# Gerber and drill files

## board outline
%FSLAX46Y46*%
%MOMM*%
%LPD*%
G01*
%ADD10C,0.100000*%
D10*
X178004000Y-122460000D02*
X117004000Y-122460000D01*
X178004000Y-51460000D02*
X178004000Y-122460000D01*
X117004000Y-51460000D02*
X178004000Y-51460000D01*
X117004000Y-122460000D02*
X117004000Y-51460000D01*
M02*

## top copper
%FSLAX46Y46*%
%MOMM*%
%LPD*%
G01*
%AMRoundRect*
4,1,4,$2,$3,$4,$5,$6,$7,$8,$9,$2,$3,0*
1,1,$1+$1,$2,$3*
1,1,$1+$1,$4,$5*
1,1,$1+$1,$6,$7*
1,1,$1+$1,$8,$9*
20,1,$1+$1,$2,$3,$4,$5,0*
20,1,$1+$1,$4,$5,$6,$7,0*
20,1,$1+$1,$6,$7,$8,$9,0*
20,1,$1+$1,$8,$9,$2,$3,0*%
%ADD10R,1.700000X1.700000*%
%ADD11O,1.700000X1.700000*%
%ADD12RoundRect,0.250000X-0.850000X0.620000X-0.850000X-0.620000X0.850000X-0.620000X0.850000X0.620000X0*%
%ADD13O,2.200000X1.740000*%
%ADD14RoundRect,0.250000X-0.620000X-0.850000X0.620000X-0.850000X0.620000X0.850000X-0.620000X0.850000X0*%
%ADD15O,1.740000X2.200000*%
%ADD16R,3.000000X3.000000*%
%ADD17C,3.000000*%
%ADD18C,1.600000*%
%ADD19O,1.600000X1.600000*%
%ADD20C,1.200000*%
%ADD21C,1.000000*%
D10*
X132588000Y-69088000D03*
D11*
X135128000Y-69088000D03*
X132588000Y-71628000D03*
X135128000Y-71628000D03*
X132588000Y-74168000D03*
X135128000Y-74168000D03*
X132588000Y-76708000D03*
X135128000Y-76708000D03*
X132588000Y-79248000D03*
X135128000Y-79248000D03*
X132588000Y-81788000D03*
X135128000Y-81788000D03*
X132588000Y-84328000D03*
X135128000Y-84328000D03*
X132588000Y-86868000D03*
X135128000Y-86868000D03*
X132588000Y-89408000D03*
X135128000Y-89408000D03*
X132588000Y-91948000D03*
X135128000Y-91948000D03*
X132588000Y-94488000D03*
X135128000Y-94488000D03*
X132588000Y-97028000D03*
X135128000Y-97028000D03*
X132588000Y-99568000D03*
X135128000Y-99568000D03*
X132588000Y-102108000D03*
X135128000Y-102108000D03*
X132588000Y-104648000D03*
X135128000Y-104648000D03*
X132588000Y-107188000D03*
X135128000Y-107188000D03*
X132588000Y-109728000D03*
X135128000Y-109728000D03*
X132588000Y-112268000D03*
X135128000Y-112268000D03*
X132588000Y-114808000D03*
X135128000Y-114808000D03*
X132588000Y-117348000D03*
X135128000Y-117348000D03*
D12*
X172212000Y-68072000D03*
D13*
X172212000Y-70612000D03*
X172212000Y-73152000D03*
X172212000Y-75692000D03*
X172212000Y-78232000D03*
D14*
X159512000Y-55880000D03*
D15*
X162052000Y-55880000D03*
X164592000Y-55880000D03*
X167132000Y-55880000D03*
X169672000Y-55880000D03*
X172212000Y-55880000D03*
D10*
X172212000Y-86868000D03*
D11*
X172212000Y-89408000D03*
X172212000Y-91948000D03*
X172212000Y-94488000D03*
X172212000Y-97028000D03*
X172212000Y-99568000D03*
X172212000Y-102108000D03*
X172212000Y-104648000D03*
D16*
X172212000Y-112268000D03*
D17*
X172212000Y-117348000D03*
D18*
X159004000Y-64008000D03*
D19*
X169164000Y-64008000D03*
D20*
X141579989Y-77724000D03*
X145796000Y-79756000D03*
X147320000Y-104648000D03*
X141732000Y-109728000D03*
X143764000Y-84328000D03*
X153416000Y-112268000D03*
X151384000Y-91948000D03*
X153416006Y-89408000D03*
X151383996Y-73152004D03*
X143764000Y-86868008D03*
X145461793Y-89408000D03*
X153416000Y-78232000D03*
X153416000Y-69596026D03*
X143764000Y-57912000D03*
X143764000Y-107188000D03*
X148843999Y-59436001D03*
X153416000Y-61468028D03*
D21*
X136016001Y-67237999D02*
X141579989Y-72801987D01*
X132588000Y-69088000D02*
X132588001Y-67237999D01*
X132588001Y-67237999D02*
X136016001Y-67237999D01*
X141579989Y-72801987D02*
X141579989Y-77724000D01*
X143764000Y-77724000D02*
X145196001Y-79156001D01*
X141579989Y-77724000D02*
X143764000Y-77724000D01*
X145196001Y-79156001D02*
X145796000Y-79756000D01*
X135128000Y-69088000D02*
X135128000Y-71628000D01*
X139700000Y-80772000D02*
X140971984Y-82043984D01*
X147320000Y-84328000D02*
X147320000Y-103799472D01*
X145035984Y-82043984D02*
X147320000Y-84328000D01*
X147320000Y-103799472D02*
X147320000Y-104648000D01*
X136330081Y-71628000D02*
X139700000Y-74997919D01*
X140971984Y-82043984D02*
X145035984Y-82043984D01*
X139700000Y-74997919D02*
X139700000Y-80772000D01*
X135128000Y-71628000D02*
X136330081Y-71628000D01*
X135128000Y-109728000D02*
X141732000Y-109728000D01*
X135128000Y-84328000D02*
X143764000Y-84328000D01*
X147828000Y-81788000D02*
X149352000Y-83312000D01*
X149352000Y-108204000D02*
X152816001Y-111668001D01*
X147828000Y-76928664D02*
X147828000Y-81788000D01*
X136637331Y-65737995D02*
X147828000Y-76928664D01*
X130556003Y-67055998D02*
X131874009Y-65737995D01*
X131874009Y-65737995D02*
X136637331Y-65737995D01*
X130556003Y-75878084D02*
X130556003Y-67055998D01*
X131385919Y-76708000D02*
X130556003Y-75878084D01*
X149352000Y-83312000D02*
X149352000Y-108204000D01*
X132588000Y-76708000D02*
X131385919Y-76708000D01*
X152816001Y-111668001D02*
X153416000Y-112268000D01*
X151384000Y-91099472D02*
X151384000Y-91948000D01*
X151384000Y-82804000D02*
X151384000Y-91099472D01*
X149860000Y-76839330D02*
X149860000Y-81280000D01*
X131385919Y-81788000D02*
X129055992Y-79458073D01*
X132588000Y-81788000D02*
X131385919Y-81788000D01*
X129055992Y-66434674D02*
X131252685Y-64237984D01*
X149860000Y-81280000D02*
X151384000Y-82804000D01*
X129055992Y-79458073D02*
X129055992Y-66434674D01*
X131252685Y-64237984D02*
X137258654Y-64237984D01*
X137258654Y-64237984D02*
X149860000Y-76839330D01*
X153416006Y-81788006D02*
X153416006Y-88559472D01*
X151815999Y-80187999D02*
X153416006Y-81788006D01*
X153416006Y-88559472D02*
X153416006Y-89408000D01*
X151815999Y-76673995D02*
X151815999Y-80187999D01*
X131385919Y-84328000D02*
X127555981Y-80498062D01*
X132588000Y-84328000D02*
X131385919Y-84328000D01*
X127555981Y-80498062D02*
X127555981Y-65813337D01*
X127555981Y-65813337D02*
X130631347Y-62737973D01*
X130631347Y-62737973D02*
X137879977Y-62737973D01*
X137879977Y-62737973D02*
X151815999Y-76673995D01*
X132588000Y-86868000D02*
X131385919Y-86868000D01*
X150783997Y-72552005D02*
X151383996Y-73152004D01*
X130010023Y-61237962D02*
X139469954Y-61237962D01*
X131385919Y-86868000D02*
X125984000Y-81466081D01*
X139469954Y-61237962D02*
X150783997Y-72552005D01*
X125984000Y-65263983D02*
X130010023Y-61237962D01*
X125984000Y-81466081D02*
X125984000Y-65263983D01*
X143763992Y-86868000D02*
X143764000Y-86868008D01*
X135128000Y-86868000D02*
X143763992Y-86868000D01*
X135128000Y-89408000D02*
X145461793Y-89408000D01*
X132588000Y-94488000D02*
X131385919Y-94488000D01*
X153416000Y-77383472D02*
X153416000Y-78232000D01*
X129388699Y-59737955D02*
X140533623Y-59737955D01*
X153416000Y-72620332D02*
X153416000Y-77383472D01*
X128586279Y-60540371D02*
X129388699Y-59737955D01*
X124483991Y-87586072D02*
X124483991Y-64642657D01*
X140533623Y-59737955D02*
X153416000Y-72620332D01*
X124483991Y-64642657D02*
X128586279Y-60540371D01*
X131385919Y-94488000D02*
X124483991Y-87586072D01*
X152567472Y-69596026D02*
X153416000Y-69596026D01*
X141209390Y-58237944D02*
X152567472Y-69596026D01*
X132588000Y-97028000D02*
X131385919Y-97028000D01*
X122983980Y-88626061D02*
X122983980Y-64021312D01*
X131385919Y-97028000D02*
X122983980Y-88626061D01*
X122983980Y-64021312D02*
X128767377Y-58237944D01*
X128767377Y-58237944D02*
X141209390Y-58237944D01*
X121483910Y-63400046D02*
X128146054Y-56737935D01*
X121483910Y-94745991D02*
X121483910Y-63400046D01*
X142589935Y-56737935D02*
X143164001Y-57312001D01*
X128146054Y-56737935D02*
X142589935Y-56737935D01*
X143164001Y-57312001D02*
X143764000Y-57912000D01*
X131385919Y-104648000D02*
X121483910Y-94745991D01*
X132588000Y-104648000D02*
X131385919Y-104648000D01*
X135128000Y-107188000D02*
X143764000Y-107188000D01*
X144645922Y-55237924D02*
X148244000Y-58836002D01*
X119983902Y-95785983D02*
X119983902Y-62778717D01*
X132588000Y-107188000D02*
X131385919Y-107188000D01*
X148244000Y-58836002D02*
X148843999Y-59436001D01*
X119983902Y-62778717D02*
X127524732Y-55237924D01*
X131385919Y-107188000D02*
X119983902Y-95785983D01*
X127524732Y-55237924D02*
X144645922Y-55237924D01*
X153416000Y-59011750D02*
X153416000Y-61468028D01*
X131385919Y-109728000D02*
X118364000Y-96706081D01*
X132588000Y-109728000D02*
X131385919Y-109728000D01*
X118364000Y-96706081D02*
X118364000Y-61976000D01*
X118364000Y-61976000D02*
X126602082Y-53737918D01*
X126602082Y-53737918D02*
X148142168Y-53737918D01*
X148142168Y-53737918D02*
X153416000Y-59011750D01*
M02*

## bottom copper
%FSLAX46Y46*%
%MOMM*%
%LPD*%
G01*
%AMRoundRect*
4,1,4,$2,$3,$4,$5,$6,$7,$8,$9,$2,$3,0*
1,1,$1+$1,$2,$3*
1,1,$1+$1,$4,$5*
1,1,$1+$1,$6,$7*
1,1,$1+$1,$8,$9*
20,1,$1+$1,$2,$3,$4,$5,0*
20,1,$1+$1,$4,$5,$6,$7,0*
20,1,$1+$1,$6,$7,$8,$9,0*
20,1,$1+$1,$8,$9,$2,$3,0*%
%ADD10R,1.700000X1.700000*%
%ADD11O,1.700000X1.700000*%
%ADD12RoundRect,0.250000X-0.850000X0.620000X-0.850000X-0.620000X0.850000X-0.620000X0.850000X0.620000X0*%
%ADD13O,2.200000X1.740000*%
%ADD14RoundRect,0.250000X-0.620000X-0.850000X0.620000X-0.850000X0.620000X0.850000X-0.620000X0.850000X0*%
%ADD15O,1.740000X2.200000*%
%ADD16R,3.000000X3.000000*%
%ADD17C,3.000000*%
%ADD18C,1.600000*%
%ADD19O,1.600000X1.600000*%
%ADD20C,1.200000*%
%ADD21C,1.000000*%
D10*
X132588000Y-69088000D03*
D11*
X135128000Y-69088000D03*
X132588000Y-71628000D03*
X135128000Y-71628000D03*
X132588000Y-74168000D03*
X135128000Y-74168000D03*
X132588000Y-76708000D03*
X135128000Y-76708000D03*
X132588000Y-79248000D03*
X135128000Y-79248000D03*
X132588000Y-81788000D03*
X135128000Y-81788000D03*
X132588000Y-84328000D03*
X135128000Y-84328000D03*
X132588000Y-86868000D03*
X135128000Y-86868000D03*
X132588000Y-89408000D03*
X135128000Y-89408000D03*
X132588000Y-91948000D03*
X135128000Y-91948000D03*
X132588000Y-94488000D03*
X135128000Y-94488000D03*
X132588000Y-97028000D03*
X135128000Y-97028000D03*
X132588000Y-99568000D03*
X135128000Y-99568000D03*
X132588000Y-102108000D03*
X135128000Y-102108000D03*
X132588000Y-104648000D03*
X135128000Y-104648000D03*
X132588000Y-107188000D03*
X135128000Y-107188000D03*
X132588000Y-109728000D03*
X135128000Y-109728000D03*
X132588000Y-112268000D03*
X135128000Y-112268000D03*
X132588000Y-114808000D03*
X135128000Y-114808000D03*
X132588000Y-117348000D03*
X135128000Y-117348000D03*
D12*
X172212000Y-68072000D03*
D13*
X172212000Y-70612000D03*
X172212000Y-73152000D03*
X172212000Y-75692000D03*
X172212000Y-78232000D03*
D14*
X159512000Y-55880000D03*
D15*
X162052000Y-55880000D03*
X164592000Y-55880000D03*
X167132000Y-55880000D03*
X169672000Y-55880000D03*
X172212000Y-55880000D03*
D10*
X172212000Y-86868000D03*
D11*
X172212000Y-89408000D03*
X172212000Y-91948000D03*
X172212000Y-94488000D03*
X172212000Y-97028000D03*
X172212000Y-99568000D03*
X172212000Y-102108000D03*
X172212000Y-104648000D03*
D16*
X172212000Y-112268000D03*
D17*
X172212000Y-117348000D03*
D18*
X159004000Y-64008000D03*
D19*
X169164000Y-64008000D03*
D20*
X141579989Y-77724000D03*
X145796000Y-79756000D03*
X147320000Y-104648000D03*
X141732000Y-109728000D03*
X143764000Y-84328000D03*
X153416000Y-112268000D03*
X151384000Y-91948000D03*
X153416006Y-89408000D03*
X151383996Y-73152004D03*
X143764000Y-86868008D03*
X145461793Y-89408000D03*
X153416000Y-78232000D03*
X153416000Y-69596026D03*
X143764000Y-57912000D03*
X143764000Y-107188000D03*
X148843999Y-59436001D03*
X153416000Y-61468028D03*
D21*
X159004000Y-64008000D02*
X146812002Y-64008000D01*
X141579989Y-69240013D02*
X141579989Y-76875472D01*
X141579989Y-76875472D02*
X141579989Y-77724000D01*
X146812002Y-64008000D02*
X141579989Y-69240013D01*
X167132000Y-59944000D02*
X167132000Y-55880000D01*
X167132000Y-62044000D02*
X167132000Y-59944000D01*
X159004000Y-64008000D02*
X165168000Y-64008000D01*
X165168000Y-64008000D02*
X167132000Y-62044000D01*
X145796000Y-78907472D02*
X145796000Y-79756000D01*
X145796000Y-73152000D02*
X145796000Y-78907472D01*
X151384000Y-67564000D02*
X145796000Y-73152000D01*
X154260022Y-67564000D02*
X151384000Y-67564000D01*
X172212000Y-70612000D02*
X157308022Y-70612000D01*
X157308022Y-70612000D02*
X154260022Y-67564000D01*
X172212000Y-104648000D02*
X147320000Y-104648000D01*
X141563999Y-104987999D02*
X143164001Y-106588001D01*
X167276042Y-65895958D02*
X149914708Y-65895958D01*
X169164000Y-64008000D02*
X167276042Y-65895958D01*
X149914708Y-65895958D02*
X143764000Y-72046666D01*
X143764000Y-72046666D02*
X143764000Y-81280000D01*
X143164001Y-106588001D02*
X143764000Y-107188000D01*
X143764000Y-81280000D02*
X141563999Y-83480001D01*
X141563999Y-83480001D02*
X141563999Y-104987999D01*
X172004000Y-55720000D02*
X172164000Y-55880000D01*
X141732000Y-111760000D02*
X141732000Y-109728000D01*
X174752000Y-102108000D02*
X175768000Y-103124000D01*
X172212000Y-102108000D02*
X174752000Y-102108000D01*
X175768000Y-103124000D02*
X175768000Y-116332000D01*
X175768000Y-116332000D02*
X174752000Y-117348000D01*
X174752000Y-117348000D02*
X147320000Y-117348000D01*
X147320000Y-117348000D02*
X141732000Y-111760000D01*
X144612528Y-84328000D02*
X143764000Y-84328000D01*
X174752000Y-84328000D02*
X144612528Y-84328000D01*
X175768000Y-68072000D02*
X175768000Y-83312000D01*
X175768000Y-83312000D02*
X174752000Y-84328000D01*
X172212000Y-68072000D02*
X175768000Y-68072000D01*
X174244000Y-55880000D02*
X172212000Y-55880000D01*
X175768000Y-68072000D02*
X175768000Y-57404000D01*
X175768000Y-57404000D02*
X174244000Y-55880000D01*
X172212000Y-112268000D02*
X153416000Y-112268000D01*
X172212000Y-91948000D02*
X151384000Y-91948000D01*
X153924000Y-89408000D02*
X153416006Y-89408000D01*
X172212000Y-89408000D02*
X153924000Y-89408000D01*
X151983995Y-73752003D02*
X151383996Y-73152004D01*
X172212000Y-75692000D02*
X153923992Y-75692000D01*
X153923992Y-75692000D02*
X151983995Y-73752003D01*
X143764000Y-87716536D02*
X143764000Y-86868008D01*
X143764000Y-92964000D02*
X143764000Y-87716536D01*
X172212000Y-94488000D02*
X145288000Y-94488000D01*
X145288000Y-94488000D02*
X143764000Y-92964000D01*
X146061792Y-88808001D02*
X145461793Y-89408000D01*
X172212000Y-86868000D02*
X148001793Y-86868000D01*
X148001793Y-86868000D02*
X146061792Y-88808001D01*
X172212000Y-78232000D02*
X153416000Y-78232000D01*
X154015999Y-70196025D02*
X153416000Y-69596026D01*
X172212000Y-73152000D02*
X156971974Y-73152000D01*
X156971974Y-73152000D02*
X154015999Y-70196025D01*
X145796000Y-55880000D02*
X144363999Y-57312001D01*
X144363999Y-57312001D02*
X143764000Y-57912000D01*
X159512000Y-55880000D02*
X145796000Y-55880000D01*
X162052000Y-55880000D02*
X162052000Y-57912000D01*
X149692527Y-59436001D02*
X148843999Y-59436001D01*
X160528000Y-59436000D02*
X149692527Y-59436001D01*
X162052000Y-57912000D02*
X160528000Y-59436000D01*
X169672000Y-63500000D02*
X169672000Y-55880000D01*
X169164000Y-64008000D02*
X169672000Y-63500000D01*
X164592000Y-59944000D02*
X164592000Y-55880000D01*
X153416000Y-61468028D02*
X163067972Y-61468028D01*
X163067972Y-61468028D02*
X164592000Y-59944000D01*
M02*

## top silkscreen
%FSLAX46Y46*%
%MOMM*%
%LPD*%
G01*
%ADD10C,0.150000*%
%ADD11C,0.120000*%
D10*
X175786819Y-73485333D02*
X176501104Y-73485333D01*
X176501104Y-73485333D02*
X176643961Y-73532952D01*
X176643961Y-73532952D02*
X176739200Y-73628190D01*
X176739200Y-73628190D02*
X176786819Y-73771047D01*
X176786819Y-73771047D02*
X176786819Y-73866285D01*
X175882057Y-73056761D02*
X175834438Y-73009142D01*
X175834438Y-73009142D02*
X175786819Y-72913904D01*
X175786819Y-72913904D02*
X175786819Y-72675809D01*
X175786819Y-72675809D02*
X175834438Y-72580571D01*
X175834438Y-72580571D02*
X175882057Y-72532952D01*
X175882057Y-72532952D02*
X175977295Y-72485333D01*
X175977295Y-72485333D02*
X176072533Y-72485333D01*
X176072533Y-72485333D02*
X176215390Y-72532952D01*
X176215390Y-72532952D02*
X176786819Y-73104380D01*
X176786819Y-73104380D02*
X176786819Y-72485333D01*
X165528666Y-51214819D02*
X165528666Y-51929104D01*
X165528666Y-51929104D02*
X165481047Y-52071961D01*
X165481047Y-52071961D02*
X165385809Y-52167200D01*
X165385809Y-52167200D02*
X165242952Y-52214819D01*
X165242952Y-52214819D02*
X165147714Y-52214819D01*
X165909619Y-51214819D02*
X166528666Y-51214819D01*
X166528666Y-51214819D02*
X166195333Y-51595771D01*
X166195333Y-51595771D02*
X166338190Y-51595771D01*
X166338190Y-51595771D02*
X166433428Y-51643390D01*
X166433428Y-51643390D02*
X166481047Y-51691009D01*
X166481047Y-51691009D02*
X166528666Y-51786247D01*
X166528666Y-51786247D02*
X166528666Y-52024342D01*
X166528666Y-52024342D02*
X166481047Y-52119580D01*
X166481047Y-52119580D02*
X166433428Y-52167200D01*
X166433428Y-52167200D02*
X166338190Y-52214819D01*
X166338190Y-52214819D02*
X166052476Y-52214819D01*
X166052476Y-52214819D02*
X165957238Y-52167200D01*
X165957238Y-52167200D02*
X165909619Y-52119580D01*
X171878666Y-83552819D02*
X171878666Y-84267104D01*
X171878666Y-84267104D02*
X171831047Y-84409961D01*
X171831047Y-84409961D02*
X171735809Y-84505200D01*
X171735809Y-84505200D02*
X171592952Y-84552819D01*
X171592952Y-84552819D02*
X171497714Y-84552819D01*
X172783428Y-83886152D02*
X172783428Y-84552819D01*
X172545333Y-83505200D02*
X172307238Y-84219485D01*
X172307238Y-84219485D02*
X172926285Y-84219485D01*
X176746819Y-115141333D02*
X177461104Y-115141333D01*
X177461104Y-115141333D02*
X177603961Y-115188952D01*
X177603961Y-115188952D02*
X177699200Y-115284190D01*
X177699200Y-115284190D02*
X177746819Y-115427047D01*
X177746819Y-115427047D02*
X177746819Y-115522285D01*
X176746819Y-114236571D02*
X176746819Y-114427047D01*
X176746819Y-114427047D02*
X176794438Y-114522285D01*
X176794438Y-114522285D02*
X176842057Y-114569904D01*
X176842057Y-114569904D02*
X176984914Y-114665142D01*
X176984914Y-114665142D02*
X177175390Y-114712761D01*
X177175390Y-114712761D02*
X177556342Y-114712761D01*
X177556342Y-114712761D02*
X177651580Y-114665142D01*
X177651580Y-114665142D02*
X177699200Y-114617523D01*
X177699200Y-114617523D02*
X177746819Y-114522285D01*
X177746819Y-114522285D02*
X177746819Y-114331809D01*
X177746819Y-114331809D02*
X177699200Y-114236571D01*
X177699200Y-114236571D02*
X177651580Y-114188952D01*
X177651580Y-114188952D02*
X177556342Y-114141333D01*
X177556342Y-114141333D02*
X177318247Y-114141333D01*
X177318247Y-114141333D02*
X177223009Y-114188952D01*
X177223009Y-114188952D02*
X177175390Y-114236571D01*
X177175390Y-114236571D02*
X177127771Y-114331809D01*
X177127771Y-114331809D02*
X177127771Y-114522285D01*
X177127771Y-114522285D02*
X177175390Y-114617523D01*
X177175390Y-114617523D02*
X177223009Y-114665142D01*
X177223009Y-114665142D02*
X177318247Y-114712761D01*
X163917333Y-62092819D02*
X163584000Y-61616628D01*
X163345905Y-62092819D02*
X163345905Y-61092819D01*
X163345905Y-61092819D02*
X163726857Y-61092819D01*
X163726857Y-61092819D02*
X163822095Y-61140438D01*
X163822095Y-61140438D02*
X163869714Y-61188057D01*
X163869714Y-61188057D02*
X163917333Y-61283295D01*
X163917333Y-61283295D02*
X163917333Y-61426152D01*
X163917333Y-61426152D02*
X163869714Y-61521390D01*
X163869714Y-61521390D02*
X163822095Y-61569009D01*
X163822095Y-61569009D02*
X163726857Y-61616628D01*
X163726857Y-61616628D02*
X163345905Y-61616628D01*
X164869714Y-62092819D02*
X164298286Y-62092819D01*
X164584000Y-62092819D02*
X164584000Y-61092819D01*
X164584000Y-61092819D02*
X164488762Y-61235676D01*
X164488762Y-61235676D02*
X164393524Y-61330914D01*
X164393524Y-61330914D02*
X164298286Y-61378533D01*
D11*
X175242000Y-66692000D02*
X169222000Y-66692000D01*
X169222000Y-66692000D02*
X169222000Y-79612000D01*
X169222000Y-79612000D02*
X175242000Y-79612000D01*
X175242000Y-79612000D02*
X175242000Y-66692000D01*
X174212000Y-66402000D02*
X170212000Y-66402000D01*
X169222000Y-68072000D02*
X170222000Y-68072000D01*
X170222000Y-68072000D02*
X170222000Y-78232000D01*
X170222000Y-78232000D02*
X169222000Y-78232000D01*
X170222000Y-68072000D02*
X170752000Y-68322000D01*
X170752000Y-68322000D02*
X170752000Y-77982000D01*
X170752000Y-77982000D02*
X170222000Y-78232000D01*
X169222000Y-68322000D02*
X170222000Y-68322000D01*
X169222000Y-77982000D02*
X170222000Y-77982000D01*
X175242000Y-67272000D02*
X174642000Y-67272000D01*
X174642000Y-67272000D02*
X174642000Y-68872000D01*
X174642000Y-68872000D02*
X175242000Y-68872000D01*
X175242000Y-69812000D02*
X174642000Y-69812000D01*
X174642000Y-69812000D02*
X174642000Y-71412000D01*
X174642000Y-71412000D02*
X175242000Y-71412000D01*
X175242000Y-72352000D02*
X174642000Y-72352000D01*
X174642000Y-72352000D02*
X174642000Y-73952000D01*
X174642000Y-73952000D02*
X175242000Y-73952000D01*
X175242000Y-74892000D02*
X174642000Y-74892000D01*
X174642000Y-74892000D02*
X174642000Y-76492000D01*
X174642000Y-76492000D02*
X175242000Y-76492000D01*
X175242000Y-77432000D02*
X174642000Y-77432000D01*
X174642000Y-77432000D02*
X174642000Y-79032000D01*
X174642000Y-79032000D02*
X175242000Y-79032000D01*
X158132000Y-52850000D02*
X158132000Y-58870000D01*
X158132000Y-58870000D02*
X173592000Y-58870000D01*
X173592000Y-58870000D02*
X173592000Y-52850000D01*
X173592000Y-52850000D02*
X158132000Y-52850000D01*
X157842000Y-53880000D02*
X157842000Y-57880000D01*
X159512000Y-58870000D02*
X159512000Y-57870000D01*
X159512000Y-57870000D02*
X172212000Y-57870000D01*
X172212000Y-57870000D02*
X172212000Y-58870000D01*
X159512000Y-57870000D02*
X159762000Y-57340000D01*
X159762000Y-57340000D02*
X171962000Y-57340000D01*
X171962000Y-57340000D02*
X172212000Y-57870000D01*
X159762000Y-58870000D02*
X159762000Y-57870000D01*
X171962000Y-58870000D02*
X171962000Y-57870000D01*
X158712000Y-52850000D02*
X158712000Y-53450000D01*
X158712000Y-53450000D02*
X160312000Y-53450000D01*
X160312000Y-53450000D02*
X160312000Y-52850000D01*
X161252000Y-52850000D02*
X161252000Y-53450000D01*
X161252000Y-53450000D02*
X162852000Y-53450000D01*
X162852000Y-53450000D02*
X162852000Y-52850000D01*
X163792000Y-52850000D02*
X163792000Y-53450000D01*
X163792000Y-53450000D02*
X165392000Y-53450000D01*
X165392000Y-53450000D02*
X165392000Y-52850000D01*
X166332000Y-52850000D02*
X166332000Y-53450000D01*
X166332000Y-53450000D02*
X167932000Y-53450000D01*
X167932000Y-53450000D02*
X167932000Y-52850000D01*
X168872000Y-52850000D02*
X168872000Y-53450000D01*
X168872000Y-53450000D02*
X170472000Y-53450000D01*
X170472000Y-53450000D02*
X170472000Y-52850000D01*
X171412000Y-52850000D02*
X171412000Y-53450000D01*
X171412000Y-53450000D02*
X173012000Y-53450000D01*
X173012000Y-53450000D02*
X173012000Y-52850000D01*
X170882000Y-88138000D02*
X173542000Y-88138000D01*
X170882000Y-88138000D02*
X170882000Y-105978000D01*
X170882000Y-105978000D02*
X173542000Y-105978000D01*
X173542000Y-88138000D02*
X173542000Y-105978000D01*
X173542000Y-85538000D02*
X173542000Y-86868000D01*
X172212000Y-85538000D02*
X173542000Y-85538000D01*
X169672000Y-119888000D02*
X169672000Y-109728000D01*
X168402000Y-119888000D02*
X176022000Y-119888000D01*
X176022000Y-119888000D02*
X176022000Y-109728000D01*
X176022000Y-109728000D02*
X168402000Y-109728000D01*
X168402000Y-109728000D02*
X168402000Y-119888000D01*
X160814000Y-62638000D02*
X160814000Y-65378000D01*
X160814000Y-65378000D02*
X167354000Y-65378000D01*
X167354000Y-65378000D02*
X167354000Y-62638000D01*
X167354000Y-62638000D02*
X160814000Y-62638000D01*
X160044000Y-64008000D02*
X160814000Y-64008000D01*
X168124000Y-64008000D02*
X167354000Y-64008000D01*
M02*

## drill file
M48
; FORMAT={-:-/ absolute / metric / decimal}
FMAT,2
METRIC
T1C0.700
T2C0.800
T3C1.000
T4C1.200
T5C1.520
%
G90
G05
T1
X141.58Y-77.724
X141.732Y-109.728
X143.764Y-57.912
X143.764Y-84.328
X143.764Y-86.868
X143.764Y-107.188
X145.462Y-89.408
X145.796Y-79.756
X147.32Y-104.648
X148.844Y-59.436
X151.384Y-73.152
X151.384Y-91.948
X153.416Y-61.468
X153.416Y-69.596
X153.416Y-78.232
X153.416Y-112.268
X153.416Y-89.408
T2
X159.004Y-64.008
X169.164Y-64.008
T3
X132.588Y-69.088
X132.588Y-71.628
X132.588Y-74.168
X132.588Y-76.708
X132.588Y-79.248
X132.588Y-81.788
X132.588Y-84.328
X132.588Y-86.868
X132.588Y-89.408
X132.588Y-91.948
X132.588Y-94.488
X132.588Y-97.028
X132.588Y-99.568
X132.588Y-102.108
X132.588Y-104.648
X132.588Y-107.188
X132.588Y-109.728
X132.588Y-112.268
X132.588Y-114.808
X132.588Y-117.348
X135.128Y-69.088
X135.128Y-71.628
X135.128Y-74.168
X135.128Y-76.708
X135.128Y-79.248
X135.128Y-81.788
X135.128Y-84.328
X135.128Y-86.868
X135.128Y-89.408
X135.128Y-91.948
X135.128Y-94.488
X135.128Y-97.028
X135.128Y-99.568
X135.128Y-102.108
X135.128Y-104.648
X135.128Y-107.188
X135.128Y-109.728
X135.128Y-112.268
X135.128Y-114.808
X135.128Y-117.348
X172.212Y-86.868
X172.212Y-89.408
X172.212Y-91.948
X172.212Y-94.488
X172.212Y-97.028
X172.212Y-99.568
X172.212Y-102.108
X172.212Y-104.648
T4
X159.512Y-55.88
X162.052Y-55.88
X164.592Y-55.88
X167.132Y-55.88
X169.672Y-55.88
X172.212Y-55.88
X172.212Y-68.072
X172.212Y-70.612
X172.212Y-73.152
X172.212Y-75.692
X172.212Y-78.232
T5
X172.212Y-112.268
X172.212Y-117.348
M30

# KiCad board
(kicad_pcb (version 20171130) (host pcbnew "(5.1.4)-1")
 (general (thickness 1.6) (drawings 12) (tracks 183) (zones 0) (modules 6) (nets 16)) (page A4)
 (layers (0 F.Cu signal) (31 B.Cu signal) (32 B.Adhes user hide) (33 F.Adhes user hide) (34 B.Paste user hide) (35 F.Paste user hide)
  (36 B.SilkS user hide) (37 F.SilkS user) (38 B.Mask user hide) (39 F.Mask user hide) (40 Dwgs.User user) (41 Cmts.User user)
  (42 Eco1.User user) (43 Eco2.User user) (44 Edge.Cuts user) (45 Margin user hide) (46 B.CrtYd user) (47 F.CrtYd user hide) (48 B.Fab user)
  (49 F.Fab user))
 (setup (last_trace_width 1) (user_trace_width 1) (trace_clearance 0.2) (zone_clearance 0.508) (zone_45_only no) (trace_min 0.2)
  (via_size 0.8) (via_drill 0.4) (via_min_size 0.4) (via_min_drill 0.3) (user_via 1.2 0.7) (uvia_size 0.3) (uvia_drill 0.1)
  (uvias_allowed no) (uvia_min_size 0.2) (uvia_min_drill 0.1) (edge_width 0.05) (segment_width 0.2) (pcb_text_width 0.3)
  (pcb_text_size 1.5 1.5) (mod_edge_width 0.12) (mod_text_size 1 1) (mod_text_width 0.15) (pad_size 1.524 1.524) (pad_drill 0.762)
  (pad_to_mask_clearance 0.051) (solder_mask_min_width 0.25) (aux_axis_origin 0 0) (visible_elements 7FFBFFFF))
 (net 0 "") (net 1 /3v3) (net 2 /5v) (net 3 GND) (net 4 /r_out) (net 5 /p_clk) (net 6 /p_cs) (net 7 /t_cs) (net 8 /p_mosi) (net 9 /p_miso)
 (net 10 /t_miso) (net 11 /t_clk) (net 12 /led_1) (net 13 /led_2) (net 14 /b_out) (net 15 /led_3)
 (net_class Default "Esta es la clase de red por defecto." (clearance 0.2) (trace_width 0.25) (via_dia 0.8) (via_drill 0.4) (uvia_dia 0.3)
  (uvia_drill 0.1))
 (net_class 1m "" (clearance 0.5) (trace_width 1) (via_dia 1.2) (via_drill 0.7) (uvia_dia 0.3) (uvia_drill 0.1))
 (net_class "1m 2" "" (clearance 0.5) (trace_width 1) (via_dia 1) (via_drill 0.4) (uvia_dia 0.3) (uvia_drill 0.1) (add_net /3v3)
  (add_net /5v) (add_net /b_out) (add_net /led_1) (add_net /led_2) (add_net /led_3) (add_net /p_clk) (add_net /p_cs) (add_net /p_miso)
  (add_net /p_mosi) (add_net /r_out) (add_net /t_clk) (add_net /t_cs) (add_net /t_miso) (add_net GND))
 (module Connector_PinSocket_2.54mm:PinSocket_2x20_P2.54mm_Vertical (layer B.Cu) (at 132.588 69.088 180)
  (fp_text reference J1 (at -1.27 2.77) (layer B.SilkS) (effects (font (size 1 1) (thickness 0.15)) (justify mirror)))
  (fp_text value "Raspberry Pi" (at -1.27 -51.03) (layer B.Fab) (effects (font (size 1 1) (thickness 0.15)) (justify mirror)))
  (pad 1 thru_hole rect (at 0 0 180) (size 1.7 1.7) (drill 1) (layers *.Cu *.Mask) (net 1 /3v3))
  (pad 2 thru_hole oval (at -2.54 0 180) (size 1.7 1.7) (drill 1) (layers *.Cu *.Mask) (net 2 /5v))
  (pad 3 thru_hole oval (at 0 -2.54 180) (size 1.7 1.7) (drill 1) (layers *.Cu *.Mask))
  (pad 4 thru_hole oval (at -2.54 -2.54 180) (size 1.7 1.7) (drill 1) (layers *.Cu *.Mask) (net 2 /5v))
  (pad 5 thru_hole oval (at 0 -5.08 180) (size 1.7 1.7) (drill 1) (layers *.Cu *.Mask))
  (pad 6 thru_hole oval (at -2.54 -5.08 180) (size 1.7 1.7) (drill 1) (layers *.Cu *.Mask) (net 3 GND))
  (pad 7 thru_hole oval (at 0 -7.62 180) (size 1.7 1.7) (drill 1) (layers *.Cu *.Mask) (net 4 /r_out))
  (pad 8 thru_hole oval (at -2.54 -7.62 180) (size 1.7 1.7) (drill 1) (layers *.Cu *.Mask))
  (pad 9 thru_hole oval (at 0 -10.16 180) (size 1.7 1.7) (drill 1) (layers *.Cu *.Mask))
  (pad 10 thru_hole oval (at -2.54 -10.16 180) (size 1.7 1.7) (drill 1) (layers *.Cu *.Mask))
  (pad 11 thru_hole oval (at 0 -12.7 180) (size 1.7 1.7) (drill 1) (layers *.Cu *.Mask) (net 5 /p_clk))
  (pad 12 thru_hole oval (at -2.54 -12.7 180) (size 1.7 1.7) (drill 1) (layers *.Cu *.Mask))
  (pad 13 thru_hole oval (at 0 -15.24 180) (size 1.7 1.7) (drill 1) (layers *.Cu *.Mask) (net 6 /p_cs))
  (pad 14 thru_hole oval (at -2.54 -15.24 180) (size 1.7 1.7) (drill 1) (layers *.Cu *.Mask) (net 3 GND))
  (pad 15 thru_hole oval (at 0 -17.78 180) (size 1.7 1.7) (drill 1) (layers *.Cu *.Mask) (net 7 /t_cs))
  (pad 16 thru_hole oval (at -2.54 -17.78 180) (size 1.7 1.7) (drill 1) (layers *.Cu *.Mask) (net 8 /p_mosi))
  (pad 17 thru_hole oval (at 0 -20.32 180) (size 1.7 1.7) (drill 1) (layers *.Cu *.Mask))
  (pad 18 thru_hole oval (at -2.54 -20.32 180) (size 1.7 1.7) (drill 1) (layers *.Cu *.Mask) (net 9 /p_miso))
  (pad 19 thru_hole oval (at 0 -22.86 180) (size 1.7 1.7) (drill 1) (layers *.Cu *.Mask))
  (pad 20 thru_hole oval (at -2.54 -22.86 180) (size 1.7 1.7) (drill 1) (layers *.Cu *.Mask) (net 3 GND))
  (pad 21 thru_hole oval (at 0 -25.4 180) (size 1.7 1.7) (drill 1) (layers *.Cu *.Mask) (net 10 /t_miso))
  (pad 22 thru_hole oval (at -2.54 -25.4 180) (size 1.7 1.7) (drill 1) (layers *.Cu *.Mask))
  (pad 23 thru_hole oval (at 0 -27.94 180) (size 1.7 1.7) (drill 1) (layers *.Cu *.Mask) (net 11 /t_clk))
  (pad 24 thru_hole oval (at -2.54 -27.94 180) (size 1.7 1.7) (drill 1) (layers *.Cu *.Mask))
  (pad 25 thru_hole oval (at 0 -30.48 180) (size 1.7 1.7) (drill 1) (layers *.Cu *.Mask))
  (pad 26 thru_hole oval (at -2.54 -30.48 180) (size 1.7 1.7) (drill 1) (layers *.Cu *.Mask))
  (pad 27 thru_hole oval (at 0 -33.02 180) (size 1.7 1.7) (drill 1) (layers *.Cu *.Mask))
  (pad 28 thru_hole oval (at -2.54 -33.02 180) (size 1.7 1.7) (drill 1) (layers *.Cu *.Mask))
  (pad 29 thru_hole oval (at 0 -35.56 180) (size 1.7 1.7) (drill 1) (layers *.Cu *.Mask) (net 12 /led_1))
  (pad 30 thru_hole oval (at -2.54 -35.56 180) (size 1.7 1.7) (drill 1) (layers *.Cu *.Mask) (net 3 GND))
  (pad 31 thru_hole oval (at 0 -38.1 180) (size 1.7 1.7) (drill 1) (layers *.Cu *.Mask) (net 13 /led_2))
  (pad 32 thru_hole oval (at -2.54 -38.1 180) (size 1.7 1.7) (drill 1) (layers *.Cu *.Mask) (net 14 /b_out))
  (pad 33 thru_hole oval (at 0 -40.64 180) (size 1.7 1.7) (drill 1) (layers *.Cu *.Mask) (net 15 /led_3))
  (pad 34 thru_hole oval (at -2.54 -40.64 180) (size 1.7 1.7) (drill 1) (layers *.Cu *.Mask) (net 3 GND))
  (pad 35 thru_hole oval (at 0 -43.18 180) (size 1.7 1.7) (drill 1) (layers *.Cu *.Mask))
  (pad 36 thru_hole oval (at -2.54 -43.18 180) (size 1.7 1.7) (drill 1) (layers *.Cu *.Mask))
  (pad 37 thru_hole oval (at 0 -45.72 180) (size 1.7 1.7) (drill 1) (layers *.Cu *.Mask))
  (pad 38 thru_hole oval (at -2.54 -45.72 180) (size 1.7 1.7) (drill 1) (layers *.Cu *.Mask))
  (pad 39 thru_hole oval (at 0 -48.26 180) (size 1.7 1.7) (drill 1) (layers *.Cu *.Mask))
  (pad 40 thru_hole oval (at -2.54 -48.26 180) (size 1.7 1.7) (drill 1) (layers *.Cu *.Mask)))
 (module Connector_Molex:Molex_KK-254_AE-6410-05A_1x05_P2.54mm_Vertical (layer F.Cu) (at 172.212 68.072 270)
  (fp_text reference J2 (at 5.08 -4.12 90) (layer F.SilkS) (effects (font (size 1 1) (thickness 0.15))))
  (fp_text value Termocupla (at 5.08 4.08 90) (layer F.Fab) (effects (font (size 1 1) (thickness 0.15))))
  (fp_line (start -1.38 -3.03) (end -1.38 2.99) (layer F.SilkS) (width 0.12))
  (fp_line (start -1.38 2.99) (end 11.54 2.99) (layer F.SilkS) (width 0.12))
  (fp_line (start 11.54 2.99) (end 11.54 -3.03) (layer F.SilkS) (width 0.12))
  (fp_line (start 11.54 -3.03) (end -1.38 -3.03) (layer F.SilkS) (width 0.12))
  (fp_line (start -1.67 -2) (end -1.67 2) (layer F.SilkS) (width 0.12))
  (fp_line (start 0 2.99) (end 0 1.99) (layer F.SilkS) (width 0.12))
  (fp_line (start 0 1.99) (end 10.16 1.99) (layer F.SilkS) (width 0.12))
  (fp_line (start 10.16 1.99) (end 10.16 2.99) (layer F.SilkS) (width 0.12))
  (fp_line (start 0 1.99) (end 0.25 1.46) (layer F.SilkS) (width 0.12))
  (fp_line (start 0.25 1.46) (end 9.91 1.46) (layer F.SilkS) (width 0.12))
  (fp_line (start 9.91 1.46) (end 10.16 1.99) (layer F.SilkS) (width 0.12))
  (fp_line (start 0.25 2.99) (end 0.25 1.99) (layer F.SilkS) (width 0.12))
  (fp_line (start 9.91 2.99) (end 9.91 1.99) (layer F.SilkS) (width 0.12))
  (fp_line (start -0.8 -3.03) (end -0.8 -2.43) (layer F.SilkS) (width 0.12))
  (fp_line (start -0.8 -2.43) (end 0.8 -2.43) (layer F.SilkS) (width 0.12))
  (fp_line (start 0.8 -2.43) (end 0.8 -3.03) (layer F.SilkS) (width 0.12))
  (fp_line (start 1.74 -3.03) (end 1.74 -2.43) (layer F.SilkS) (width 0.12))
  (fp_line (start 1.74 -2.43) (end 3.34 -2.43) (layer F.SilkS) (width 0.12))
  (fp_line (start 3.34 -2.43) (end 3.34 -3.03) (layer F.SilkS) (width 0.12))
  (fp_line (start 4.28 -3.03) (end 4.28 -2.43) (layer F.SilkS) (width 0.12))
  (fp_line (start 4.28 -2.43) (end 5.88 -2.43) (layer F.SilkS) (width 0.12))
  (fp_line (start 5.88 -2.43) (end 5.88 -3.03) (layer F.SilkS) (width 0.12))
  (fp_line (start 6.82 -3.03) (end 6.82 -2.43) (layer F.SilkS) (width 0.12))
  (fp_line (start 6.82 -2.43) (end 8.42 -2.43) (layer F.SilkS) (width 0.12))
  (fp_line (start 8.42 -2.43) (end 8.42 -3.03) (layer F.SilkS) (width 0.12))
  (fp_line (start 9.36 -3.03) (end 9.36 -2.43) (layer F.SilkS) (width 0.12))
  (fp_line (start 9.36 -2.43) (end 10.96 -2.43) (layer F.SilkS) (width 0.12))
  (fp_line (start 10.96 -2.43) (end 10.96 -3.03) (layer F.SilkS) (width 0.12))
  (pad 1 thru_hole roundrect (at 0 0 270) (size 1.74 2.2) (drill 1.2) (layers *.Cu *.Mask) (roundrect_rratio 0.143678) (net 3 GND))
  (pad 2 thru_hole oval (at 2.54 0 270) (size 1.74 2.2) (drill 1.2) (layers *.Cu *.Mask) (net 1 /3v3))
  (pad 3 thru_hole oval (at 5.08 0 270) (size 1.74 2.2) (drill 1.2) (layers *.Cu *.Mask) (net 11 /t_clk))
  (pad 4 thru_hole oval (at 7.62 0 270) (size 1.74 2.2) (drill 1.2) (layers *.Cu *.Mask) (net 7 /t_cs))
  (pad 5 thru_hole oval (at 10.16 0 270) (size 1.74 2.2) (drill 1.2) (layers *.Cu *.Mask) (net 10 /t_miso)))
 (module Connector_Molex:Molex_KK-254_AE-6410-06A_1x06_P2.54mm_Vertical (layer F.Cu) (at 159.512 55.88)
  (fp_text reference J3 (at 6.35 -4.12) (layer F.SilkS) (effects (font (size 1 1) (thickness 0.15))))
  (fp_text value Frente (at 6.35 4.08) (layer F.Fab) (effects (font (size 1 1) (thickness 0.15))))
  (fp_line (start -1.38 -3.03) (end -1.38 2.99) (layer F.SilkS) (width 0.12))
  (fp_line (start -1.38 2.99) (end 14.08 2.99) (layer F.SilkS) (width 0.12))
  (fp_line (start 14.08 2.99) (end 14.08 -3.03) (layer F.SilkS) (width 0.12))
  (fp_line (start 14.08 -3.03) (end -1.38 -3.03) (layer F.SilkS) (width 0.12))
  (fp_line (start -1.67 -2) (end -1.67 2) (layer F.SilkS) (width 0.12))
  (fp_line (start 0 2.99) (end 0 1.99) (layer F.SilkS) (width 0.12))
  (fp_line (start 0 1.99) (end 12.7 1.99) (layer F.SilkS) (width 0.12))
  (fp_line (start 12.7 1.99) (end 12.7 2.99) (layer F.SilkS) (width 0.12))
  (fp_line (start 0 1.99) (end 0.25 1.46) (layer F.SilkS) (width 0.12))
  (fp_line (start 0.25 1.46) (end 12.45 1.46) (layer F.SilkS) (width 0.12))
  (fp_line (start 12.45 1.46) (end 12.7 1.99) (layer F.SilkS) (width 0.12))
  (fp_line (start 0.25 2.99) (end 0.25 1.99) (layer F.SilkS) (width 0.12))
  (fp_line (start 12.45 2.99) (end 12.45 1.99) (layer F.SilkS) (width 0.12))
  (fp_line (start -0.8 -3.03) (end -0.8 -2.43) (layer F.SilkS) (width 0.12))
  (fp_line (start -0.8 -2.43) (end 0.8 -2.43) (layer F.SilkS) (width 0.12))
  (fp_line (start 0.8 -2.43) (end 0.8 -3.03) (layer F.SilkS) (width 0.12))
  (fp_line (start 1.74 -3.03) (end 1.74 -2.43) (layer F.SilkS) (width 0.12))
  (fp_line (start 1.74 -2.43) (end 3.34 -2.43) (layer F.SilkS) (width 0.12))
  (fp_line (start 3.34 -2.43) (end 3.34 -3.03) (layer F.SilkS) (width 0.12))
  (fp_line (start 4.28 -3.03) (end 4.28 -2.43) (layer F.SilkS) (width 0.12))
  (fp_line (start 4.28 -2.43) (end 5.88 -2.43) (layer F.SilkS) (width 0.12))
  (fp_line (start 5.88 -2.43) (end 5.88 -3.03) (layer F.SilkS) (width 0.12))
  (fp_line (start 6.82 -3.03) (end 6.82 -2.43) (layer F.SilkS) (width 0.12))
  (fp_line (start 6.82 -2.43) (end 8.42 -2.43) (layer F.SilkS) (width 0.12))
  (fp_line (start 8.42 -2.43) (end 8.42 -3.03) (layer F.SilkS) (width 0.12))
  (fp_line (start 9.36 -3.03) (end 9.36 -2.43) (layer F.SilkS) (width 0.12))
  (fp_line (start 9.36 -2.43) (end 10.96 -2.43) (layer F.SilkS) (width 0.12))
  (fp_line (start 10.96 -2.43) (end 10.96 -3.03) (layer F.SilkS) (width 0.12))
  (fp_line (start 11.9 -3.03) (end 11.9 -2.43) (layer F.SilkS) (width 0.12))
  (fp_line (start 11.9 -2.43) (end 13.5 -2.43) (layer F.SilkS) (width 0.12))
  (fp_line (start 13.5 -2.43) (end 13.5 -3.03) (layer F.SilkS) (width 0.12))
  (pad 1 thru_hole roundrect (at 0 0) (size 1.74 2.2) (drill 1.2) (layers *.Cu *.Mask) (roundrect_rratio 0.143678) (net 12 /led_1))
  (pad 2 thru_hole oval (at 2.54 0) (size 1.74 2.2) (drill 1.2) (layers *.Cu *.Mask) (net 13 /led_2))
  (pad 3 thru_hole oval (at 5.08 0) (size 1.74 2.2) (drill 1.2) (layers *.Cu *.Mask) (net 15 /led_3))
  (pad 4 thru_hole oval (at 7.62 0) (size 1.74 2.2) (drill 1.2) (layers *.Cu *.Mask) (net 1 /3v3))
  (pad 5 thru_hole oval (at 10.16 0) (size 1.74 2.2) (drill 1.2) (layers *.Cu *.Mask) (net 14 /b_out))
  (pad 6 thru_hole oval (at 12.7 0) (size 1.74 2.2) (drill 1.2) (layers *.Cu *.Mask) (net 3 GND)))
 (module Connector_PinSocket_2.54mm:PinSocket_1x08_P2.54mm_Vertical (layer F.Cu) (at 172.212 86.868)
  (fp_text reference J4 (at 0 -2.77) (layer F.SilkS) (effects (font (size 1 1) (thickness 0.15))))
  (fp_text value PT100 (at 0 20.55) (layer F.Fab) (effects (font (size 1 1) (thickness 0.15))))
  (fp_line (start -1.33 1.27) (end 1.33 1.27) (layer F.SilkS) (width 0.12))
  (fp_line (start -1.33 1.27) (end -1.33 19.11) (layer F.SilkS) (width 0.12))
  (fp_line (start -1.33 19.11) (end 1.33 19.11) (layer F.SilkS) (width 0.12))
  (fp_line (start 1.33 1.27) (end 1.33 19.11) (layer F.SilkS) (width 0.12))
  (fp_line (start 1.33 -1.33) (end 1.33 0) (layer F.SilkS) (width 0.12))
  (fp_line (start 0 -1.33) (end 1.33 -1.33) (layer F.SilkS) (width 0.12))
  (pad 1 thru_hole rect (at 0 0) (size 1.7 1.7) (drill 1) (layers *.Cu *.Mask) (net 9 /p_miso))
  (pad 2 thru_hole oval (at 0 2.54) (size 1.7 1.7) (drill 1) (layers *.Cu *.Mask) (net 6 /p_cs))
  (pad 3 thru_hole oval (at 0 5.08) (size 1.7 1.7) (drill 1) (layers *.Cu *.Mask) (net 5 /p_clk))
  (pad 4 thru_hole oval (at 0 7.62) (size 1.7 1.7) (drill 1) (layers *.Cu *.Mask) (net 8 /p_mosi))
  (pad 5 thru_hole oval (at 0 10.16) (size 1.7 1.7) (drill 1) (layers *.Cu *.Mask))
  (pad 6 thru_hole oval (at 0 12.7) (size 1.7 1.7) (drill 1) (layers *.Cu *.Mask))
  (pad 7 thru_hole oval (at 0 15.24) (size 1.7 1.7) (drill 1) (layers *.Cu *.Mask) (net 3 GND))
  (pad 8 thru_hole oval (at 0 17.78) (size 1.7 1.7) (drill 1) (layers *.Cu *.Mask) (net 2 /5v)))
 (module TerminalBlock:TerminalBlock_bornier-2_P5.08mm (layer F.Cu) (at 172.212 112.268 270)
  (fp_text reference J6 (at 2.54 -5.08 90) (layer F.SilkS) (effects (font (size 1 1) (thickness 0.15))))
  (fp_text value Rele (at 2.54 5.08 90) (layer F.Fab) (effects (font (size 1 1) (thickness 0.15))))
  (fp_line (start 7.62 2.54) (end -2.54 2.54) (layer F.SilkS) (width 0.12))
  (fp_line (start 7.62 3.81) (end 7.62 -3.81) (layer F.SilkS) (width 0.12))
  (fp_line (start 7.62 -3.81) (end -2.54 -3.81) (layer F.SilkS) (width 0.12))
  (fp_line (start -2.54 -3.81) (end -2.54 3.81) (layer F.SilkS) (width 0.12))
  (fp_line (start -2.54 3.81) (end 7.62 3.81) (layer F.SilkS) (width 0.12))
  (pad 1 thru_hole rect (at 0 0 270) (size 3 3) (drill 1.52) (layers *.Cu *.Mask) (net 4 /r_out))
  (pad 2 thru_hole circle (at 5.08 0 270) (size 3 3) (drill 1.52) (layers *.Cu *.Mask) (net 3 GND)))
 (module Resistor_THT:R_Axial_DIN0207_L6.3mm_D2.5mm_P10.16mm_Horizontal (layer F.Cu) (at 159.004 64.008)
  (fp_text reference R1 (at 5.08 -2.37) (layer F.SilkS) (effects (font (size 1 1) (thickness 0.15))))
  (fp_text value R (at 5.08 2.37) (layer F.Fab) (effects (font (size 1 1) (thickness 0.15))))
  (fp_line (start 1.81 -1.37) (end 1.81 1.37) (layer F.SilkS) (width 0.12))
  (fp_line (start 1.81 1.37) (end 8.35 1.37) (layer F.SilkS) (width 0.12))
  (fp_line (start 8.35 1.37) (end 8.35 -1.37) (layer F.SilkS) (width 0.12))
  (fp_line (start 8.35 -1.37) (end 1.81 -1.37) (layer F.SilkS) (width 0.12))
  (fp_line (start 1.04 0) (end 1.81 0) (layer F.SilkS) (width 0.12))
  (fp_line (start 9.12 0) (end 8.35 0) (layer F.SilkS) (width 0.12))
  (pad 1 thru_hole circle (at 0 0) (size 1.6 1.6) (drill 0.8) (layers *.Cu *.Mask) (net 1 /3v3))
  (pad 2 thru_hole oval (at 10.16 0) (size 1.6 1.6) (drill 0.8) (layers *.Cu *.Mask) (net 14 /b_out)))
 (gr_line (start 178.004 122.46) (end 117.004 122.46) (layer Edge.Cuts) (width 0.1))
 (gr_line (start 178.004 51.46) (end 178.004 122.46) (layer Edge.Cuts) (width 0.1))
 (gr_line (start 117.004 51.46) (end 178.004 51.46) (layer Edge.Cuts) (width 0.1))
 (gr_line (start 117.004 122.46) (end 117.004 51.46) (layer Edge.Cuts) (width 0.1))
 (segment (start 136.016001 67.237999) (end 141.579989 72.801987) (width 1) (layer F.Cu) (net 1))
 (segment (start 159.004 64.008) (end 146.812002 64.008) (width 1) (layer B.Cu) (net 1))
 (segment (start 141.579989 69.240013) (end 141.579989 76.875472) (width 1) (layer B.Cu) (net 1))
 (segment (start 141.579989 76.875472) (end 141.579989 77.724) (width 1) (layer B.Cu) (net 1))
 (segment (start 132.588 69.088) (end 132.588001 67.237999) (width 1) (layer F.Cu) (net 1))
 (segment (start 132.588001 67.237999) (end 136.016001 67.237999) (width 1) (layer F.Cu) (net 1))
 (segment (start 141.579989 72.801987) (end 141.579989 77.724) (width 1) (layer F.Cu) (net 1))
 (segment (start 146.812002 64.008) (end 141.579989 69.240013) (width 1) (layer B.Cu) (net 1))
 (via (at 141.579989 77.724) (size 1.2) (drill 0.7) (layers F.Cu B.Cu) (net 1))
 (via (at 145.796 79.756) (size 1.2) (drill 0.7) (layers F.Cu B.Cu) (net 1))
 (segment (start 143.764 77.724) (end 145.196001 79.156001) (width 1) (layer F.Cu) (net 1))
 (segment (start 141.579989 77.724) (end 143.764 77.724) (width 1) (layer F.Cu) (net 1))
 (segment (start 145.196001 79.156001) (end 145.796 79.756) (width 1) (layer F.Cu) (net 1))
 (segment (start 167.132 59.944) (end 167.132 55.88) (width 1) (layer B.Cu) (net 1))
 (segment (start 167.132 62.044) (end 167.132 59.944) (width 1) (layer B.Cu) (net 1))
 (segment (start 159.004 64.008) (end 165.168 64.008) (width 1) (layer B.Cu) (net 1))
 (segment (start 165.168 64.008) (end 167.132 62.044) (width 1) (layer B.Cu) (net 1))
 (segment (start 145.796 78.907472) (end 145.796 79.756) (width 1) (layer B.Cu) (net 1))
 (segment (start 145.796 73.152) (end 145.796 78.907472) (width 1) (layer B.Cu) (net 1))
 (segment (start 151.384 67.564) (end 145.796 73.152) (width 1) (layer B.Cu) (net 1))
 (segment (start 154.260022 67.564) (end 151.384 67.564) (width 1) (layer B.Cu) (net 1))
 (segment (start 172.212 70.612) (end 157.308022 70.612) (width 1) (layer B.Cu) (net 1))
 (segment (start 157.308022 70.612) (end 154.260022 67.564) (width 1) (layer B.Cu) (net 1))
 (segment (start 135.128 69.088) (end 135.128 71.628) (width 1) (layer F.Cu) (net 2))
 (via (at 147.32 104.648) (size 1.2) (drill 0.7) (layers F.Cu B.Cu) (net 2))
 (segment (start 139.7 80.772) (end 140.971984 82.043984) (width 1) (layer F.Cu) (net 2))
 (segment (start 147.32 84.328) (end 147.32 103.799472) (width 1) (layer F.Cu) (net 2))
 (segment (start 172.212 104.648) (end 147.32 104.648) (width 1) (layer B.Cu) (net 2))
 (segment (start 145.035984 82.043984) (end 147.32 84.328) (width 1) (layer F.Cu) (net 2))
 (segment (start 147.32 103.799472) (end 147.32 104.648) (width 1) (layer F.Cu) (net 2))
 (segment (start 136.330081 71.628) (end 139.7 74.997919) (width 1) (layer F.Cu) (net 2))
 (segment (start 140.971984 82.043984) (end 145.035984 82.043984) (width 1) (layer F.Cu) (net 2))
 (segment (start 139.7 74.997919) (end 139.7 80.772) (width 1) (layer F.Cu) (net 2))
 (segment (start 135.128 71.628) (end 136.330081 71.628) (width 1) (layer F.Cu) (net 2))
 (via (at 141.732 109.728) (size 1.2) (drill 0.7) (layers F.Cu B.Cu) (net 3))
 (segment (start 135.128 109.728) (end 141.732 109.728) (width 1) (layer F.Cu) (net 3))
 (via (at 143.764 84.328) (size 1.2) (drill 0.7) (layers F.Cu B.Cu) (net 3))
 (segment (start 135.128 84.328) (end 143.764 84.328) (width 1) (layer F.Cu) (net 3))
 (segment (start 147.828 81.788) (end 149.352 83.312) (width 1) (layer F.Cu) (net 4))
 (segment (start 149.352 108.204) (end 152.816001 111.668001) (width 1) (layer F.Cu) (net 4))
 (segment (start 147.828 76.928664) (end 147.828 81.788) (width 1) (layer F.Cu) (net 4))
 (segment (start 136.637331 65.737995) (end 147.828 76.928664) (width 1) (layer F.Cu) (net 4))
 (segment (start 130.556003 67.055998) (end 131.874009 65.737995) (width 1) (layer F.Cu) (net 4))
 (segment (start 131.874009 65.737995) (end 136.637331 65.737995) (width 1) (layer F.Cu) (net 4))
 (segment (start 130.556003 75.878084) (end 130.556003 67.055998) (width 1) (layer F.Cu) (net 4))
 (segment (start 131.385919 76.708) (end 130.556003 75.878084) (width 1) (layer F.Cu) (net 4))
 (segment (start 149.352 83.312) (end 149.352 108.204) (width 1) (layer F.Cu) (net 4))
 (segment (start 132.588 76.708) (end 131.385919 76.708) (width 1) (layer F.Cu) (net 4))
 (via (at 153.416 112.268) (size 1.2) (drill 0.7) (layers F.Cu B.Cu) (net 4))
 (segment (start 152.816001 111.668001) (end 153.416 112.268) (width 1) (layer F.Cu) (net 4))
 (via (at 151.384 91.948) (size 1.2) (drill 0.7) (layers F.Cu B.Cu) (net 5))
 (segment (start 151.384 91.099472) (end 151.384 91.948) (width 1) (layer F.Cu) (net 5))
 (segment (start 151.384 82.804) (end 151.384 91.099472) (width 1) (layer F.Cu) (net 5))
 (segment (start 149.86 76.83933) (end 149.86 81.28) (width 1) (layer F.Cu) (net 5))
 (segment (start 131.385919 81.788) (end 129.055992 79.458073) (width 1) (layer F.Cu) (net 5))
 (segment (start 132.588 81.788) (end 131.385919 81.788) (width 1) (layer F.Cu) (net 5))
 (segment (start 129.055992 66.434674) (end 131.252685 64.237984) (width 1) (layer F.Cu) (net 5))
 (segment (start 149.86 81.28) (end 151.384 82.804) (width 1) (layer F.Cu) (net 5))
 (segment (start 129.055992 79.458073) (end 129.055992 66.434674) (width 1) (layer F.Cu) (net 5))
 (segment (start 131.252685 64.237984) (end 137.258654 64.237984) (width 1) (layer F.Cu) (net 5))
 (segment (start 137.258654 64.237984) (end 149.86 76.83933) (width 1) (layer F.Cu) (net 5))
 (via (at 153.416006 89.408) (size 1.2) (drill 0.7) (layers F.Cu B.Cu) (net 6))
 (segment (start 153.416006 81.788006) (end 153.416006 88.559472) (width 1) (layer F.Cu) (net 6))
 (segment (start 151.815999 80.187999) (end 153.416006 81.788006) (width 1) (layer F.Cu) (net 6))
 (segment (start 153.416006 88.559472) (end 153.416006 89.408) (width 1) (layer F.Cu) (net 6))
 (segment (start 151.815999 76.673995) (end 151.815999 80.187999) (width 1) (layer F.Cu) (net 6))
 (segment (start 131.385919 84.328) (end 127.555981 80.498062) (width 1) (layer F.Cu) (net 6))
 (segment (start 132.588 84.328) (end 131.385919 84.328) (width 1) (layer F.Cu) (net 6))
 (segment (start 127.555981 80.498062) (end 127.555981 65.813337) (width 1) (layer F.Cu) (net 6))
 (segment (start 127.555981 65.813337) (end 130.631347 62.737973) (width 1) (layer F.Cu) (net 6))
 (segment (start 130.631347 62.737973) (end 137.879977 62.737973) (width 1) (layer F.Cu) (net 6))
 (segment (start 137.879977 62.737973) (end 151.815999 76.673995) (width 1) (layer F.Cu) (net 6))
 (segment (start 132.588 86.868) (end 131.385919 86.868) (width 1) (layer F.Cu) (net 7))
 (segment (start 150.783997 72.552005) (end 151.383996 73.152004) (width 1) (layer F.Cu) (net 7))
 (segment (start 130.010023 61.237962) (end 139.469954 61.237962) (width 1) (layer F.Cu) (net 7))
 (segment (start 131.385919 86.868) (end 125.984 81.466081) (width 1) (layer F.Cu) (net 7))
 (segment (start 139.469954 61.237962) (end 150.783997 72.552005) (width 1) (layer F.Cu) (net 7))
 (segment (start 125.984 65.263983) (end 130.010023 61.237962) (width 1) (layer F.Cu) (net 7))
 (segment (start 125.984 81.466081) (end 125.984 65.263983) (width 1) (layer F.Cu) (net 7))
 (via (at 151.383996 73.152004) (size 1.2) (drill 0.7) (layers F.Cu B.Cu) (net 7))
 (segment (start 143.763992 86.868) (end 143.764 86.868008) (width 1) (layer F.Cu) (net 8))
 (segment (start 135.128 86.868) (end 143.763992 86.868) (width 1) (layer F.Cu) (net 8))
 (via (at 143.764 86.868008) (size 1.2) (drill 0.7) (layers F.Cu B.Cu) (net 8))
 (via (at 145.461793 89.408) (size 1.2) (drill 0.7) (layers F.Cu B.Cu) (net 9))
 (segment (start 135.128 89.408) (end 145.461793 89.408) (width 1) (layer F.Cu) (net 9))
 (segment (start 132.588 94.488) (end 131.385919 94.488) (width 1) (layer F.Cu) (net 10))
 (via (at 153.416 78.232) (size 1.2) (drill 0.7) (layers F.Cu B.Cu) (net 10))
 (segment (start 153.416 77.383472) (end 153.416 78.232) (width 1) (layer F.Cu) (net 10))
 (segment (start 129.388699 59.737955) (end 140.533623 59.737955) (width 1) (layer F.Cu) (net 10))
 (segment (start 153.416 72.620332) (end 153.416 77.383472) (width 1) (layer F.Cu) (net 10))
 (segment (start 128.586279 60.540371) (end 129.388699 59.737955) (width 1) (layer F.Cu) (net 10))
 (segment (start 124.483991 87.586072) (end 124.483991 64.642657) (width 1) (layer F.Cu) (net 10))
 (segment (start 140.533623 59.737955) (end 153.416 72.620332) (width 1) (layer F.Cu) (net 10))
 (segment (start 124.483991 64.642657) (end 128.586279 60.540371) (width 1) (layer F.Cu) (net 10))
 (segment (start 131.385919 94.488) (end 124.483991 87.586072) (width 1) (layer F.Cu) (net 10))
 (via (at 153.416 69.596026) (size 1.2) (drill 0.7) (layers F.Cu B.Cu) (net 11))
 (segment (start 152.567472 69.596026) (end 153.416 69.596026) (width 1) (layer F.Cu) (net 11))
 (segment (start 141.20939 58.237944) (end 152.567472 69.596026) (width 1) (layer F.Cu) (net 11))
 (segment (start 132.588 97.028) (end 131.385919 97.028) (width 1) (layer F.Cu) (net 11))
 (segment (start 122.98398 88.626061) (end 122.98398 64.021312) (width 1) (layer F.Cu) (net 11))
 (segment (start 131.385919 97.028) (end 122.98398 88.626061) (width 1) (layer F.Cu) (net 11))
 (segment (start 122.98398 64.021312) (end 128.767377 58.237944) (width 1) (layer F.Cu) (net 11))
 (segment (start 128.767377 58.237944) (end 141.20939 58.237944) (width 1) (layer F.Cu) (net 11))
 (via (at 143.764 57.912) (size 1.2) (drill 0.7) (layers F.Cu B.Cu) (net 12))
 (segment (start 121.48391 63.400046) (end 128.146054 56.737935) (width 1) (layer F.Cu) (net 12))
 (segment (start 121.48391 94.745991) (end 121.48391 63.400046) (width 1) (layer F.Cu) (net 12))
 (segment (start 142.589935 56.737935) (end 143.164001 57.312001) (width 1) (layer F.Cu) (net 12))
 (segment (start 128.146054 56.737935) (end 142.589935 56.737935) (width 1) (layer F.Cu) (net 12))
 (segment (start 143.164001 57.312001) (end 143.764 57.912) (width 1) (layer F.Cu) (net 12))
 (segment (start 131.385919 104.648) (end 121.48391 94.745991) (width 1) (layer F.Cu) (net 12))
 (segment (start 132.588 104.648) (end 131.385919 104.648) (width 1) (layer F.Cu) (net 12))
 (segment (start 135.128 107.188) (end 143.764 107.188) (width 1) (layer F.Cu) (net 14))
 (via (at 143.764 107.188) (size 1.2) (drill 0.7) (layers F.Cu B.Cu) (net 14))
 (segment (start 141.563999 104.987999) (end 143.164001 106.588001) (width 1) (layer B.Cu) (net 14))
 (segment (start 167.276042 65.895958) (end 149.914708 65.895958) (width 1) (layer B.Cu) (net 14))
 (segment (start 169.164 64.008) (end 167.276042 65.895958) (width 1) (layer B.Cu) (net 14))
 (segment (start 149.914708 65.895958) (end 143.764 72.046666) (width 1) (layer B.Cu) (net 14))
 (segment (start 143.764 72.046666) (end 143.764 81.28) (width 1) (layer B.Cu) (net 14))
 (segment (start 143.164001 106.588001) (end 143.764 107.188) (width 1) (layer B.Cu) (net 14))
 (segment (start 143.764 81.28) (end 141.563999 83.480001) (width 1) (layer B.Cu) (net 14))
 (segment (start 141.563999 83.480001) (end 141.563999 104.987999) (width 1) (layer B.Cu) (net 14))
 (segment (start 172.004 55.72) (end 172.164 55.88) (width 1) (layer B.Cu) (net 3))
 (segment (start 141.732 111.76) (end 141.732 109.728) (width 1) (layer B.Cu) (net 3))
 (segment (start 174.752 102.108) (end 175.768 103.124) (width 1) (layer B.Cu) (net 3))
 (segment (start 172.212 102.108) (end 174.752 102.108) (width 1) (layer B.Cu) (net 3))
 (segment (start 175.768 103.124) (end 175.768 116.332) (width 1) (layer B.Cu) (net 3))
 (segment (start 175.768 116.332) (end 174.752 117.348) (width 1) (layer B.Cu) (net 3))
 (segment (start 174.752 117.348) (end 147.32 117.348) (width 1) (layer B.Cu) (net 3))
 (segment (start 147.32 117.348) (end 141.732 111.76) (width 1) (layer B.Cu) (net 3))
 (segment (start 144.612528 84.328) (end 143.764 84.328) (width 1) (layer B.Cu) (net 3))
 (segment (start 174.752 84.328) (end 144.612528 84.328) (width 1) (layer B.Cu) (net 3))
 (segment (start 175.768 68.072) (end 175.768 83.312) (width 1) (layer B.Cu) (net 3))
 (segment (start 175.768 83.312) (end 174.752 84.328) (width 1) (layer B.Cu) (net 3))
 (segment (start 172.212 68.072) (end 175.768 68.072) (width 1) (layer B.Cu) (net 3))
 (segment (start 174.244 55.88) (end 172.212 55.88) (width 1) (layer B.Cu) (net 3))
 (segment (start 175.768 68.072) (end 175.768 57.404) (width 1) (layer B.Cu) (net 3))
 (segment (start 175.768 57.404) (end 174.244 55.88) (width 1) (layer B.Cu) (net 3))
 (segment (start 172.212 112.268) (end 153.416 112.268) (width 1) (layer B.Cu) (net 4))
 (segment (start 172.212 91.948) (end 151.384 91.948) (width 1) (layer B.Cu) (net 5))
 (segment (start 153.924 89.408) (end 153.416006 89.408) (width 1) (layer B.Cu) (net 6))
 (segment (start 172.212 89.408) (end 153.924 89.408) (width 1) (layer B.Cu) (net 6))
 (segment (start 151.983995 73.752003) (end 151.383996 73.152004) (width 1) (layer B.Cu) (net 7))
 (segment (start 172.212 75.692) (end 153.923992 75.692) (width 1) (layer B.Cu) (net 7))
 (segment (start 153.923992 75.692) (end 151.983995 73.752003) (width 1) (layer B.Cu) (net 7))
 (segment (start 143.764 87.716536) (end 143.764 86.868008) (width 1) (layer B.Cu) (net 8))
 (segment (start 143.764 92.964) (end 143.764 87.716536) (width 1) (layer B.Cu) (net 8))
 (segment (start 172.212 94.488) (end 145.288 94.488) (width 1) (layer B.Cu) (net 8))
 (segment (start 145.288 94.488) (end 143.764 92.964) (width 1) (layer B.Cu) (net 8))
 (segment (start 146.061792 88.808001) (end 145.461793 89.408) (width 1) (layer B.Cu) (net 9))
 (segment (start 172.212 86.868) (end 148.001793 86.868) (width 1) (layer B.Cu) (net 9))
 (segment (start 148.001793 86.868) (end 146.061792 88.808001) (width 1) (layer B.Cu) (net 9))
 (segment (start 172.212 78.232) (end 153.416 78.232) (width 1) (layer B.Cu) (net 10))
 (segment (start 154.015999 70.196025) (end 153.416 69.596026) (width 1) (layer B.Cu) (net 11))
 (segment (start 172.212 73.152) (end 156.971974 73.152) (width 1) (layer B.Cu) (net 11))
 (segment (start 156.971974 73.152) (end 154.015999 70.196025) (width 1) (layer B.Cu) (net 11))
 (segment (start 145.796 55.88) (end 144.363999 57.312001) (width 1) (layer B.Cu) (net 12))
 (segment (start 144.363999 57.312001) (end 143.764 57.912) (width 1) (layer B.Cu) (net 12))
 (segment (start 159.512 55.88) (end 145.796 55.88) (width 1) (layer B.Cu) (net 12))
 (segment (start 144.645922 55.237924) (end 148.244 58.836002) (width 1) (layer F.Cu) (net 13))
 (segment (start 119.983902 95.785983) (end 119.983902 62.778717) (width 1) (layer F.Cu) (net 13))
 (segment (start 132.588 107.188) (end 131.385919 107.188) (width 1) (layer F.Cu) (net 13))
 (segment (start 148.244 58.836002) (end 148.843999 59.436001) (width 1) (layer F.Cu) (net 13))
 (segment (start 119.983902 62.778717) (end 127.524732 55.237924) (width 1) (layer F.Cu) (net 13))
 (segment (start 131.385919 107.188) (end 119.983902 95.785983) (width 1) (layer F.Cu) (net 13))
 (segment (start 127.524732 55.237924) (end 144.645922 55.237924) (width 1) (layer F.Cu) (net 13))
 (via (at 148.843999 59.436001) (size 1.2) (drill 0.7) (layers F.Cu B.Cu) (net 13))
 (segment (start 162.052 55.88) (end 162.052 57.912) (width 1) (layer B.Cu) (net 13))
 (segment (start 149.692527 59.436001) (end 148.843999 59.436001) (width 1) (layer B.Cu) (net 13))
 (segment (start 160.528 59.436) (end 149.692527 59.436001) (width 1) (layer B.Cu) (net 13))
 (segment (start 162.052 57.912) (end 160.528 59.436) (width 1) (layer B.Cu) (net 13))
 (segment (start 169.672 63.5) (end 169.672 55.88) (width 1) (layer B.Cu) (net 14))
 (segment (start 169.164 64.008) (end 169.672 63.5) (width 1) (layer B.Cu) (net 14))
 (via (at 153.416 61.468028) (size 1.2) (drill 0.7) (layers F.Cu B.Cu) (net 15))
 (segment (start 153.416 59.01175) (end 153.416 61.468028) (width 1) (layer F.Cu) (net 15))
 (segment (start 131.385919 109.728) (end 118.364 96.706081) (width 1) (layer F.Cu) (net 15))
 (segment (start 132.588 109.728) (end 131.385919 109.728) (width 1) (layer F.Cu) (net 15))
 (segment (start 118.364 96.706081) (end 118.364 61.976) (width 1) (layer F.Cu) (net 15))
 (segment (start 118.364 61.976) (end 126.602082 53.737918) (width 1) (layer F.Cu) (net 15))
 (segment (start 126.602082 53.737918) (end 148.142168 53.737918) (width 1) (layer F.Cu) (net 15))
 (segment (start 148.142168 53.737918) (end 153.416 59.01175) (width 1) (layer F.Cu) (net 15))
 (segment (start 164.592 59.944) (end 164.592 55.88) (width 1) (layer B.Cu) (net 15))
 (segment (start 153.416 61.468028) (end 163.067972 61.468028) (width 1) (layer B.Cu) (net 15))
 (segment (start 163.067972 61.468028) (end 164.592 59.944) (width 1) (layer B.Cu) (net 15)))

